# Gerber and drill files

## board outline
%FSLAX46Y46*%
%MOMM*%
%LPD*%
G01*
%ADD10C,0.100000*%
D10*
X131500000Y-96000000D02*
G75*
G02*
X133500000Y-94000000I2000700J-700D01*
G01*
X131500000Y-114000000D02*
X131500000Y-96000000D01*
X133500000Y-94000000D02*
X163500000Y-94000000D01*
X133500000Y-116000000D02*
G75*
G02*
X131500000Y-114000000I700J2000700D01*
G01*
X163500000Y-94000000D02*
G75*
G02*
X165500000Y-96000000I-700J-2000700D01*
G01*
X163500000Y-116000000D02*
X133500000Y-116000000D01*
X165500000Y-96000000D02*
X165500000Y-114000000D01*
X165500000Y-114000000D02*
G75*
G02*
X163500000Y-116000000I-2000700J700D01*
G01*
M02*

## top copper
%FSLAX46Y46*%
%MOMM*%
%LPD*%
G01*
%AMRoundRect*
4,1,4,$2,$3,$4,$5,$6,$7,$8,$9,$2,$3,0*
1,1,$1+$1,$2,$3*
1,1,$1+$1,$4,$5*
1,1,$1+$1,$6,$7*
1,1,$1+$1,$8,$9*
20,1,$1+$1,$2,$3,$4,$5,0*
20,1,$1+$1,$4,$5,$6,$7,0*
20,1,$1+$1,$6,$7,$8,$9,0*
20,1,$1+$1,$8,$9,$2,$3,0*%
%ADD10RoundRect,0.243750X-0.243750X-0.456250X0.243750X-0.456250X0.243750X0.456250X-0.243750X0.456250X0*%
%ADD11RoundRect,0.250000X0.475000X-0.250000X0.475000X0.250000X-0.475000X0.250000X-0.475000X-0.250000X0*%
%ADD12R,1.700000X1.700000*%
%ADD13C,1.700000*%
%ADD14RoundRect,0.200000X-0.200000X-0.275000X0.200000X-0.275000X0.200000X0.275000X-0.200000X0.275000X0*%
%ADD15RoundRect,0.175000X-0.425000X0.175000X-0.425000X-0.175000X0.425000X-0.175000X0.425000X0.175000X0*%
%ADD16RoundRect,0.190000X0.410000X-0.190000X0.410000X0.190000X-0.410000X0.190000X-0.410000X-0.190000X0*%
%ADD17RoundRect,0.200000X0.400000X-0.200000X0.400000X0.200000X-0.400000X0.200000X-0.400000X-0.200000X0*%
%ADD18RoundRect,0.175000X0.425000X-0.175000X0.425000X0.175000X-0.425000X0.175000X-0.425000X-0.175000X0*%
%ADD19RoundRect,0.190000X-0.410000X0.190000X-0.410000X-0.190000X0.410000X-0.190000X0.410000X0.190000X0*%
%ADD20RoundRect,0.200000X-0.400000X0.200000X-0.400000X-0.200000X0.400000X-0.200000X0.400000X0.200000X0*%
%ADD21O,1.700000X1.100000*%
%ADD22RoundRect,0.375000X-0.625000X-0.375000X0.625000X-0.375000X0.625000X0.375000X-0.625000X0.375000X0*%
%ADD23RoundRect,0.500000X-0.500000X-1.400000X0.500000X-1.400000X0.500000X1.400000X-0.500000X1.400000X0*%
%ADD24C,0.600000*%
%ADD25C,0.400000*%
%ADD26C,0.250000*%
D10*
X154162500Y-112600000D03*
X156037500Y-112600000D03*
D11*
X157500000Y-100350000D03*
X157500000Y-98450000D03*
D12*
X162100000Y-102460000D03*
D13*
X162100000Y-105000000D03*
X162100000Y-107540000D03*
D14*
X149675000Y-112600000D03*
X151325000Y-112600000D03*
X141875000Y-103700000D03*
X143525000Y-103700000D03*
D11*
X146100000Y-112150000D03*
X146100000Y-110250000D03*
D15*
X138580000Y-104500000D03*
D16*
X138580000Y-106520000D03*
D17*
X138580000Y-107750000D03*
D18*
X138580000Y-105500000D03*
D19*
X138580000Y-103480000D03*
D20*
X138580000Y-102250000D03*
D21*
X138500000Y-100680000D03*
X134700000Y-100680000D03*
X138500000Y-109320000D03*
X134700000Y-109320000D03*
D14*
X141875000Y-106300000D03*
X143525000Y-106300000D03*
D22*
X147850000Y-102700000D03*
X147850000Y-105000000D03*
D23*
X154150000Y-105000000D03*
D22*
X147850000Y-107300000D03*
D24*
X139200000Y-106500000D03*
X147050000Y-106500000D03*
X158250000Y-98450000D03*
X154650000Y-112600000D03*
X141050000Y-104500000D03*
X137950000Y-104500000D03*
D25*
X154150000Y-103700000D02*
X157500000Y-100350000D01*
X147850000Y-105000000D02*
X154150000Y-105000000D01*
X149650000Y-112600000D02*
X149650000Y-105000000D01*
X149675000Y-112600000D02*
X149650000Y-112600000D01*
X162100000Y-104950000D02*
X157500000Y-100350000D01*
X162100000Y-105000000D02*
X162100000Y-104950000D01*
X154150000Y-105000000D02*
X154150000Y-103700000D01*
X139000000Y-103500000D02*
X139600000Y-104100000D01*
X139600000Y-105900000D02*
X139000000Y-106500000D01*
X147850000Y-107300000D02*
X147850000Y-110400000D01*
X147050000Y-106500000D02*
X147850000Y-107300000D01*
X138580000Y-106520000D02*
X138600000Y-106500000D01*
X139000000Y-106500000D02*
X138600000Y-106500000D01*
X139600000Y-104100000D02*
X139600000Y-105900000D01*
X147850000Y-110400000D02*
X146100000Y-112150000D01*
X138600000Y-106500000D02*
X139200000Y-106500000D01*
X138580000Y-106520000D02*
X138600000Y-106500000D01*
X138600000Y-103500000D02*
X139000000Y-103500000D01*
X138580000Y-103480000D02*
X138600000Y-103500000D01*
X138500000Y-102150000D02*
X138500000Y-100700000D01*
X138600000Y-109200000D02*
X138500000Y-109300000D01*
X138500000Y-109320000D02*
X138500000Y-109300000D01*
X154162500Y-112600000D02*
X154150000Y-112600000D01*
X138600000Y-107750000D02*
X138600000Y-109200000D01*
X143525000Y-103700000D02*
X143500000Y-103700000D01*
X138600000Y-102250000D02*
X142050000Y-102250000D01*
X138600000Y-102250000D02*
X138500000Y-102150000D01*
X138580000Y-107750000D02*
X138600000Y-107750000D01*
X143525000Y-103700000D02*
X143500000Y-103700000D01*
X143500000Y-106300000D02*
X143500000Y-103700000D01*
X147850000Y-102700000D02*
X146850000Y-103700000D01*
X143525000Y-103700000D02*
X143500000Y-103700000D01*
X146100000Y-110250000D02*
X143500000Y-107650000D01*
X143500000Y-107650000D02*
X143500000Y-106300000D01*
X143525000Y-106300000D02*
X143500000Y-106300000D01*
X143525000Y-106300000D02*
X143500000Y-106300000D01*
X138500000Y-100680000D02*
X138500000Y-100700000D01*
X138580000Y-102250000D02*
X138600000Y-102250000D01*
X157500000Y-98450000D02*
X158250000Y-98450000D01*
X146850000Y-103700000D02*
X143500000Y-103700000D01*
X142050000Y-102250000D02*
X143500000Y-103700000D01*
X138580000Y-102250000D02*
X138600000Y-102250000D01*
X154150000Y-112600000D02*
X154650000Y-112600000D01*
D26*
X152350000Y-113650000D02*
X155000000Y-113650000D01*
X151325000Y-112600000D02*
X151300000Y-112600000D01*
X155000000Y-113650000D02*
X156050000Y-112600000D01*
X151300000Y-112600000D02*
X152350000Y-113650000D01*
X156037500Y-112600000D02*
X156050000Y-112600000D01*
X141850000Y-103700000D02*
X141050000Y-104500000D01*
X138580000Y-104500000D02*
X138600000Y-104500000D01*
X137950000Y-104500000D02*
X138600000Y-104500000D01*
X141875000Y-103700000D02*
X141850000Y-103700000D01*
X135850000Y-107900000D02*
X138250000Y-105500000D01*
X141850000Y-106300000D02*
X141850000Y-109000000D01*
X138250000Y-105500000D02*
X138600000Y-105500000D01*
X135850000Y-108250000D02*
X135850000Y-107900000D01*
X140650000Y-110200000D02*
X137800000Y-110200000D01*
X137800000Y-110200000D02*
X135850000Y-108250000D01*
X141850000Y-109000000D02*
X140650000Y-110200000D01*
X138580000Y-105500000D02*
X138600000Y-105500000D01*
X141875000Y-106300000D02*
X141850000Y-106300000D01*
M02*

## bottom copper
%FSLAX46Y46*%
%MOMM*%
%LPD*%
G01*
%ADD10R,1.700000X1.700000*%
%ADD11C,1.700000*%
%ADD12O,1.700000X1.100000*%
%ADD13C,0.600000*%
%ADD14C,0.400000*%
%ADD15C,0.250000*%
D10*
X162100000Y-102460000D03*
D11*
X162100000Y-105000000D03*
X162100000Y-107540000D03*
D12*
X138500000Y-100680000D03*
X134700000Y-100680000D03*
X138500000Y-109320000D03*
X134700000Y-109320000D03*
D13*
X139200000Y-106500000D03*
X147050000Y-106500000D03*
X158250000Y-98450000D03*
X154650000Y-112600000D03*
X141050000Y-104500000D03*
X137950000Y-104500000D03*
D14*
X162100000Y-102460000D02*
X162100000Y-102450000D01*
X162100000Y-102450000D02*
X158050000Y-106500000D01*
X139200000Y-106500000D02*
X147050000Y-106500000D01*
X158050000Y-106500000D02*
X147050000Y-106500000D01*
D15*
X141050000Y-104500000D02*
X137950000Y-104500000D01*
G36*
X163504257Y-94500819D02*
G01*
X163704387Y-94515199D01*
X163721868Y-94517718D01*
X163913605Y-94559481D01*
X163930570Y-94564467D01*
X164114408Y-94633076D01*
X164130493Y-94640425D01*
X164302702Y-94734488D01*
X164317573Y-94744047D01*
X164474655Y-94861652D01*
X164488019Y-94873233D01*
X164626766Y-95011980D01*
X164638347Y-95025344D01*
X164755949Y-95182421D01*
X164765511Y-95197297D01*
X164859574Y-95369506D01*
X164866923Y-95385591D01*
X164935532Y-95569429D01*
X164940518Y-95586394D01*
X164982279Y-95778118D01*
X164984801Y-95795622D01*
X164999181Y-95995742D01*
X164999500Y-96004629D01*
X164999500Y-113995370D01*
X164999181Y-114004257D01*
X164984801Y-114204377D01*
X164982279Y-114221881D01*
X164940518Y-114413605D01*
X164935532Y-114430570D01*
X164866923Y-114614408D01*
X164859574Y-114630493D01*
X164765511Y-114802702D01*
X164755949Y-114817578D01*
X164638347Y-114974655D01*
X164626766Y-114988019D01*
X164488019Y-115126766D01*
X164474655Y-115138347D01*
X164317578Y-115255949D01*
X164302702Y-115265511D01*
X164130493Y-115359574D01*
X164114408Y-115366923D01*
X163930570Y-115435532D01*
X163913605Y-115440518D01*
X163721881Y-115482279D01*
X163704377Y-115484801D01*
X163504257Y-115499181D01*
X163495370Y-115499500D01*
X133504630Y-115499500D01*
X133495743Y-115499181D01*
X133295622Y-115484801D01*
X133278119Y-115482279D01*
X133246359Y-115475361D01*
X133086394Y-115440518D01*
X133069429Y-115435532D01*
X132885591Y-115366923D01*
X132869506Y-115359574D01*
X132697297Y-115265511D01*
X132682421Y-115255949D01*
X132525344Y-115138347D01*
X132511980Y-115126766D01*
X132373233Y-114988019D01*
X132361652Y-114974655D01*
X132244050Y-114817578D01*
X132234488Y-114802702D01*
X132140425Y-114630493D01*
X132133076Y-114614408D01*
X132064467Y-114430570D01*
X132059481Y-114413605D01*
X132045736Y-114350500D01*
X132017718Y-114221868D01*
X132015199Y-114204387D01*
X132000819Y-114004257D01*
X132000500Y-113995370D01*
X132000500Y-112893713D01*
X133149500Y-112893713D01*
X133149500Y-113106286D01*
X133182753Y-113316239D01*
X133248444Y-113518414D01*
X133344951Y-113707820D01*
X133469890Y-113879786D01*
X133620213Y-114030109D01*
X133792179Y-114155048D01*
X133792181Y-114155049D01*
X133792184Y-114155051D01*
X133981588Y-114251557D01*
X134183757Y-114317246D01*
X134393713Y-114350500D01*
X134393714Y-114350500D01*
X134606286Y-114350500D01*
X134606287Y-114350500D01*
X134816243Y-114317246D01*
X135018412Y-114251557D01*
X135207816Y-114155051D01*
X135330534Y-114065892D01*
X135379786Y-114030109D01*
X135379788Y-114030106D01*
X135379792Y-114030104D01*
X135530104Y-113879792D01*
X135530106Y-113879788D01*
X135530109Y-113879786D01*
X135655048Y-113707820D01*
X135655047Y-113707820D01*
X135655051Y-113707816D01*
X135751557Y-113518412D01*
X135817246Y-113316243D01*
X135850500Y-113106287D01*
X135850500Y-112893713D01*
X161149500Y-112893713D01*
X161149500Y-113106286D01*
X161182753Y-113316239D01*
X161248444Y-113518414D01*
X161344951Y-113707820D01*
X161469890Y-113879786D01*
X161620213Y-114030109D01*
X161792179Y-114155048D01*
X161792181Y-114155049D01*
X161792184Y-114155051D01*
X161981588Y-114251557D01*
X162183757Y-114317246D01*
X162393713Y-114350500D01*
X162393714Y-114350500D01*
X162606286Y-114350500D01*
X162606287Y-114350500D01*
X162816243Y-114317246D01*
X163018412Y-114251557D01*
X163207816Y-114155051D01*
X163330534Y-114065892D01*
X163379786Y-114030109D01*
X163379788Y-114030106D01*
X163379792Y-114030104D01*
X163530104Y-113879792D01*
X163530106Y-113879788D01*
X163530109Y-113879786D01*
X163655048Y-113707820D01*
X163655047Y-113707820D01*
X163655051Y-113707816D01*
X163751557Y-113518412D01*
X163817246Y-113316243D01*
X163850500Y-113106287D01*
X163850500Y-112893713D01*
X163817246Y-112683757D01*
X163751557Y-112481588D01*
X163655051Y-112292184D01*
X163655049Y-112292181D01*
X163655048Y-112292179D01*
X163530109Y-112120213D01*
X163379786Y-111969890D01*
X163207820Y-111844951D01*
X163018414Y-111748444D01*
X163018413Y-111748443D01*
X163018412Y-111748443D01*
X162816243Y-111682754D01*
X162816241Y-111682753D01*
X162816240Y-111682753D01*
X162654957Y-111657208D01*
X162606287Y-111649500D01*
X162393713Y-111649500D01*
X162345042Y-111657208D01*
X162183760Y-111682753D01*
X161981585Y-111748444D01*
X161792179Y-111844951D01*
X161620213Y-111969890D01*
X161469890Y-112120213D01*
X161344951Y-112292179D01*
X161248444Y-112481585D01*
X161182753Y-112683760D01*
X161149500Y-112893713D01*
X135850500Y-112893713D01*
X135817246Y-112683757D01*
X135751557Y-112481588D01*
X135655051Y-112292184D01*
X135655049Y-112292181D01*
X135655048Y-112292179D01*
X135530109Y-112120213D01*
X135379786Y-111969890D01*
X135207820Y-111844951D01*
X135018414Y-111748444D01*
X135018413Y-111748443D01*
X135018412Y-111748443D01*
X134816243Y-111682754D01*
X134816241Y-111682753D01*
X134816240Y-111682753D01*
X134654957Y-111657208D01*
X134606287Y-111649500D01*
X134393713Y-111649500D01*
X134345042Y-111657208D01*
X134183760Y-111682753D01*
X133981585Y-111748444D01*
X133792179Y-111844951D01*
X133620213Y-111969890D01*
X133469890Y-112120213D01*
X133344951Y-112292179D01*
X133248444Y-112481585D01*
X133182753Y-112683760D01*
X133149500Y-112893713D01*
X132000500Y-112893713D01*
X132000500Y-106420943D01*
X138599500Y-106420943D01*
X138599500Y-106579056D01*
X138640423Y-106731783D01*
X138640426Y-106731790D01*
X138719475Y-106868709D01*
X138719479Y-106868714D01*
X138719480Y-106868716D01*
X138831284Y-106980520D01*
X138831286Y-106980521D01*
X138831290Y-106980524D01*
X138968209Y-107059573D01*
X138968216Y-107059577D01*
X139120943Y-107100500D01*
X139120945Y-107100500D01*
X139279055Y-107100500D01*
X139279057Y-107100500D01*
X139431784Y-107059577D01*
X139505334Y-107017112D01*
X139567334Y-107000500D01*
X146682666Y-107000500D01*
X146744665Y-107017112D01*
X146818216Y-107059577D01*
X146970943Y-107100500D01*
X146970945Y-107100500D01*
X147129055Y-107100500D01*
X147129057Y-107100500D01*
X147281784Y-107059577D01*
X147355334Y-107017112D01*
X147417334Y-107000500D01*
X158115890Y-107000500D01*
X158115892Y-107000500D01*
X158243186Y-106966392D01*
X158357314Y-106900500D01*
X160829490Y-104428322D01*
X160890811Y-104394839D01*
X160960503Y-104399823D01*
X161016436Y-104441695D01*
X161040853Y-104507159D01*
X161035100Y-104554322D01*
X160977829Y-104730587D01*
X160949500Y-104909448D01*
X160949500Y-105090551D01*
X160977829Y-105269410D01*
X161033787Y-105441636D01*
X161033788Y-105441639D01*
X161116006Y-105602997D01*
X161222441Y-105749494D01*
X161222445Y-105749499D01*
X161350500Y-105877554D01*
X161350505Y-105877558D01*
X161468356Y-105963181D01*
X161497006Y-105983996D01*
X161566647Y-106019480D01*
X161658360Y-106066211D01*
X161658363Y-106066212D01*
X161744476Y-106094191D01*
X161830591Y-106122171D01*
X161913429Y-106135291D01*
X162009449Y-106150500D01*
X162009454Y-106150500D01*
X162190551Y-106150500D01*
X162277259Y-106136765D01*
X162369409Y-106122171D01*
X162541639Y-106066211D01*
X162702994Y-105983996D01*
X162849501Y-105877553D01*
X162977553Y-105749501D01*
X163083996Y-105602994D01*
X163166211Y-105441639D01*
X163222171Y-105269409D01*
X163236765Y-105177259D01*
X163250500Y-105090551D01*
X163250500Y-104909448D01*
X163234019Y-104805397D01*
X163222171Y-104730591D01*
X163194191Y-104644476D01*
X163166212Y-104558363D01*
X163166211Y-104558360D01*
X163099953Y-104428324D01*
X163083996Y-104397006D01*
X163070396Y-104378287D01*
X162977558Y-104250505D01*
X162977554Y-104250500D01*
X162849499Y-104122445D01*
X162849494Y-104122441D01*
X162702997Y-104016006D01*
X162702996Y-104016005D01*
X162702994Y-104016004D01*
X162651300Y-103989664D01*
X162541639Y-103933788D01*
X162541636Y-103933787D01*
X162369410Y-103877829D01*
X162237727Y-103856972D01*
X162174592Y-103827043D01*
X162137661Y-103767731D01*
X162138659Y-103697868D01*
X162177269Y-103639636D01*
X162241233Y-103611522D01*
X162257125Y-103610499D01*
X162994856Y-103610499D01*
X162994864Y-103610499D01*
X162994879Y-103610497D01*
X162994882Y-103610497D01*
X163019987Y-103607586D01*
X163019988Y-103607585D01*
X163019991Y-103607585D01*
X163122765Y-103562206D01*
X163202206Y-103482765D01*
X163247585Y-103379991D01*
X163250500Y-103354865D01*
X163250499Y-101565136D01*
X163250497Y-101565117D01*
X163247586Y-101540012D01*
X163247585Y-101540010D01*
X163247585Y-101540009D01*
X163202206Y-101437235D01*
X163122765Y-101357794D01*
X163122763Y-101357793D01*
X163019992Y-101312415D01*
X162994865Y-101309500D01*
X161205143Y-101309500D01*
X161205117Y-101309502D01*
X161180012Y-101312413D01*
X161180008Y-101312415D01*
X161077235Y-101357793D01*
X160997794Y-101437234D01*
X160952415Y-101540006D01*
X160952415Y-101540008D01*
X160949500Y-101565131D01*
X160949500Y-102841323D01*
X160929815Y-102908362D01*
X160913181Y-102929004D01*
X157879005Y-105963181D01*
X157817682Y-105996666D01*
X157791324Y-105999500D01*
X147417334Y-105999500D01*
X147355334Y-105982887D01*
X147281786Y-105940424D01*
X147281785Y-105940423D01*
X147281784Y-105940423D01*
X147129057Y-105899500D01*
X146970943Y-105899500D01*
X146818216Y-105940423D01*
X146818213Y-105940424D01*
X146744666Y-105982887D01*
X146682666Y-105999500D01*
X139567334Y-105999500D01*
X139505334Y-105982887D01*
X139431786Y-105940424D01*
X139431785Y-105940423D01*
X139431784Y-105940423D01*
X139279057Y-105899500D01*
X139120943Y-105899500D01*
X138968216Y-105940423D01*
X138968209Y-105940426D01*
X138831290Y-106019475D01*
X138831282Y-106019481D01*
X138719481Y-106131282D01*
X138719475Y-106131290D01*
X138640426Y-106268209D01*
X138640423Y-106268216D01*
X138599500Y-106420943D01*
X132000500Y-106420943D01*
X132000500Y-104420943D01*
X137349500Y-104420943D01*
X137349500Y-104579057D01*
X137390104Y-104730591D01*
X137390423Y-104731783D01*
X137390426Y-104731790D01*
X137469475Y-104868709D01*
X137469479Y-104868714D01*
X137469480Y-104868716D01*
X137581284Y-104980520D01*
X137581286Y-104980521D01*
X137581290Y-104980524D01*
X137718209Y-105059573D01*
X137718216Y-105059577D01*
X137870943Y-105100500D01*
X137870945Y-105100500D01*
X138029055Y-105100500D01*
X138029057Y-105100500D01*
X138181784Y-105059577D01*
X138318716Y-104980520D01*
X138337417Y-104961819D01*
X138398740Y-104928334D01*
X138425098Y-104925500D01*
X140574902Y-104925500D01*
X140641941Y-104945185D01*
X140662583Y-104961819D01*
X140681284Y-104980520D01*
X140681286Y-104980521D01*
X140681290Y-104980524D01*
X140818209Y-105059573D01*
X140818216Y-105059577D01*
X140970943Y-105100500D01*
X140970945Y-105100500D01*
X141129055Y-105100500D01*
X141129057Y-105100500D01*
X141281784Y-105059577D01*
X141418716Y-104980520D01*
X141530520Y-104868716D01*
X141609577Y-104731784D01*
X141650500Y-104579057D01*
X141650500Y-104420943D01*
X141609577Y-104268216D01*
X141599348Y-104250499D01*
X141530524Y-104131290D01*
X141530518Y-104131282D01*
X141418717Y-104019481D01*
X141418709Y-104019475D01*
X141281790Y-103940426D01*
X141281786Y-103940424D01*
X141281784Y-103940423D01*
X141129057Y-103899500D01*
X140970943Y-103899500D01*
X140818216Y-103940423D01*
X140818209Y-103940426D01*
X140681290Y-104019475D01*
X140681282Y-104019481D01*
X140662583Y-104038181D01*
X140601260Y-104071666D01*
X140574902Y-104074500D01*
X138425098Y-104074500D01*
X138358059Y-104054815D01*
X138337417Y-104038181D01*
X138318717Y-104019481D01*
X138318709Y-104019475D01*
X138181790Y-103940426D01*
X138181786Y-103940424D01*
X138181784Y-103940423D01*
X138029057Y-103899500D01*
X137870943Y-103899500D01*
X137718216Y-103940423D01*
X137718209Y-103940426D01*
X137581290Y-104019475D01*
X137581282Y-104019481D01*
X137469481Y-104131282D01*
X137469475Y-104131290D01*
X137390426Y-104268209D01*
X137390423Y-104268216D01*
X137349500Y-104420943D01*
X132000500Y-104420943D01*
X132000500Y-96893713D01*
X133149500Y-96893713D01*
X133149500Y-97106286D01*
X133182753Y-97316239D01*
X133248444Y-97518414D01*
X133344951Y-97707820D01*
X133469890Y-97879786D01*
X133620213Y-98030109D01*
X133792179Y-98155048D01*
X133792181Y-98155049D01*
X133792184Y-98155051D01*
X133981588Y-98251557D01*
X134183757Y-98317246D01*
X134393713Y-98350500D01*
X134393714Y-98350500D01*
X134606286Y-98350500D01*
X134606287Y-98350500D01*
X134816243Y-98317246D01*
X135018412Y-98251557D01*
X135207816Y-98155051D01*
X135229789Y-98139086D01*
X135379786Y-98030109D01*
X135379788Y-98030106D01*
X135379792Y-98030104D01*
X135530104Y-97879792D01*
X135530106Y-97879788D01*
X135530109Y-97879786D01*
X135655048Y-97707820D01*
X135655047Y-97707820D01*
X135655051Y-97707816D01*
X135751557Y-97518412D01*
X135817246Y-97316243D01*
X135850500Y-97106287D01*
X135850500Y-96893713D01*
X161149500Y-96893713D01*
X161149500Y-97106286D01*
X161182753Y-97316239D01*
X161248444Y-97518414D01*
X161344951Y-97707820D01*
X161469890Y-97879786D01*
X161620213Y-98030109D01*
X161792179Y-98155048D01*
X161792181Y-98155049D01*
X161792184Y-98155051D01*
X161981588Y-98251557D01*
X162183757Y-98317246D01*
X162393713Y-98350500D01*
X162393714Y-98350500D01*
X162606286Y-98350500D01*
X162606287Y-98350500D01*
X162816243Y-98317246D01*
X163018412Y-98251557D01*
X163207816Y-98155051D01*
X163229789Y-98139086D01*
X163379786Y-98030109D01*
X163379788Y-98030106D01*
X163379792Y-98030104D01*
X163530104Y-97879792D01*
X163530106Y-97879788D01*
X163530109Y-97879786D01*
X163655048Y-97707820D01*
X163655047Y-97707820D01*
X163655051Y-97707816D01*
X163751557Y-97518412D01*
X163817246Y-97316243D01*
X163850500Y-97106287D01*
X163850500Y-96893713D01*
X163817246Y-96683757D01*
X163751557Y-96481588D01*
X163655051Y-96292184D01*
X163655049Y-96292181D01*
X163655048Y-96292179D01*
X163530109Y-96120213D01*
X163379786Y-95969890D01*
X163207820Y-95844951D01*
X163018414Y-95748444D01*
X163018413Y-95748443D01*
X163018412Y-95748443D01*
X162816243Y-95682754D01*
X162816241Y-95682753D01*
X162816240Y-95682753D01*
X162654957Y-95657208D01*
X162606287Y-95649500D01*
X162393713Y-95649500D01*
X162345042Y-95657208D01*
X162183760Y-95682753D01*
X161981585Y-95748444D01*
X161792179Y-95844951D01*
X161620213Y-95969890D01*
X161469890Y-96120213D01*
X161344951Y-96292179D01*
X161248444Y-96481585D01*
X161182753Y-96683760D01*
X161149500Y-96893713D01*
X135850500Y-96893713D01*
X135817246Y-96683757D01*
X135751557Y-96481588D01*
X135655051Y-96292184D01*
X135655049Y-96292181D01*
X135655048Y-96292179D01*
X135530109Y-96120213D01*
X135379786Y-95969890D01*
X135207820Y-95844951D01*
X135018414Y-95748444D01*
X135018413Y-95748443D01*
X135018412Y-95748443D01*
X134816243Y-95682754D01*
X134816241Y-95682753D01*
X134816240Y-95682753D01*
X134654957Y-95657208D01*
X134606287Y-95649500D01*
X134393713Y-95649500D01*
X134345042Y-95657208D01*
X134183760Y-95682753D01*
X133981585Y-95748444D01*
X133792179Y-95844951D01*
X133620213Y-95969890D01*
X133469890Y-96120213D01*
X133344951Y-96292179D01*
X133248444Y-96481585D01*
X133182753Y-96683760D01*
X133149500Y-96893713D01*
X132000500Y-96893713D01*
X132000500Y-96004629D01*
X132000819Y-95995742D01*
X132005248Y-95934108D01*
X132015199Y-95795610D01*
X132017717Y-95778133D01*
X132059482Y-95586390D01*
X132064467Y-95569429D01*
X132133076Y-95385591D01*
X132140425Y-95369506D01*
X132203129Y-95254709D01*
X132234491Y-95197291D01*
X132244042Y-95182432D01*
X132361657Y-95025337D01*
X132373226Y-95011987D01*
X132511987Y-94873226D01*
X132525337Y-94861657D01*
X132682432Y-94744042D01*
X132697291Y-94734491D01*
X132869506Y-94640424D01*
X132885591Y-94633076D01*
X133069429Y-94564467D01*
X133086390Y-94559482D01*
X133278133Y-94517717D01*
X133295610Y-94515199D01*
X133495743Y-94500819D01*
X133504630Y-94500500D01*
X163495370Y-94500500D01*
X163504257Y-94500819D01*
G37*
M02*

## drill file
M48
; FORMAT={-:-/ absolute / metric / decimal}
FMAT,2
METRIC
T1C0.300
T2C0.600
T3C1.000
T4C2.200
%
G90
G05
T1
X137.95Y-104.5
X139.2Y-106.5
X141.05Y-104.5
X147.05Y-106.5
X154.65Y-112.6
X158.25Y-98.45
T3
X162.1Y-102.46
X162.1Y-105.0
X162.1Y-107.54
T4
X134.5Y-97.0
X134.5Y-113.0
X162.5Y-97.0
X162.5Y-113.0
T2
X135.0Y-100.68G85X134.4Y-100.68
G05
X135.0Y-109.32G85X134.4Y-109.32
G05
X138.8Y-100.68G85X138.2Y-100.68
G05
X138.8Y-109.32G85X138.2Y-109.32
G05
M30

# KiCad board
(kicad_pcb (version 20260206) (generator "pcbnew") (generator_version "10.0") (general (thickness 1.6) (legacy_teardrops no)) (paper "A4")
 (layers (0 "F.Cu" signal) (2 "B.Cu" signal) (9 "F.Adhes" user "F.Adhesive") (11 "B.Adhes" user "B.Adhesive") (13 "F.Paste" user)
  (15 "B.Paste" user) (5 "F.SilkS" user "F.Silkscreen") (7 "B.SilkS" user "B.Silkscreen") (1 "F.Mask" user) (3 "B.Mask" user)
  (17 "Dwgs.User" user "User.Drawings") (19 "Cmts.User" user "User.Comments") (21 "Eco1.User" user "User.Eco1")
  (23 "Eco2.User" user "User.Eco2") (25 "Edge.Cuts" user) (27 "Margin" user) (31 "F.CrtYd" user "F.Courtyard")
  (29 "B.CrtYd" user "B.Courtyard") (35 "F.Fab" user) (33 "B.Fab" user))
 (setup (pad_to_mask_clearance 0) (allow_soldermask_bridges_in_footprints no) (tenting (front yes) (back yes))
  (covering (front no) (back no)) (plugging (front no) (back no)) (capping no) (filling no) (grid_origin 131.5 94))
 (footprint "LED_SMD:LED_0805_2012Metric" (layer "F.Cu") (at 155.1 112.6)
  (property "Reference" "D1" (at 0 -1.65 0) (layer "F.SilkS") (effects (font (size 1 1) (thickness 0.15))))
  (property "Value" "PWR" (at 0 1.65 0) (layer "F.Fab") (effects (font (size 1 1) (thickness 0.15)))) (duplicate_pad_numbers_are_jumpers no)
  (pad "1" smd roundrect (at -0.9375 0) (size 0.975 1.4) (layers "F.Cu" "F.Mask" "F.Paste") (roundrect_rratio 0.25) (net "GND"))
  (pad "2" smd roundrect (at 0.9375 0) (size 0.975 1.4) (layers "F.Cu" "F.Mask" "F.Paste") (roundrect_rratio 0.25) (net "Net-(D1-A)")))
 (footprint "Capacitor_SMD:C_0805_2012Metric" (layer "F.Cu") (at 157.5 99.4 90)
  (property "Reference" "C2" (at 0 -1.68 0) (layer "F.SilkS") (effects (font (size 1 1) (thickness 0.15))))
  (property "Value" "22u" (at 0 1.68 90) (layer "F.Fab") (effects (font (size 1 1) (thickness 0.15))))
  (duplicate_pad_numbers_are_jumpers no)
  (pad "1" smd roundrect (at -0.95 0 90) (size 1 1.45) (layers "F.Cu" "F.Mask" "F.Paste") (roundrect_rratio 0.25) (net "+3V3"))
  (pad "2" smd roundrect (at 0.95 0 90) (size 1 1.45) (layers "F.Cu" "F.Mask" "F.Paste") (roundrect_rratio 0.25) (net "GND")))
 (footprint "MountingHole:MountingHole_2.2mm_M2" (layer "F.Cu") (at 162.5 97)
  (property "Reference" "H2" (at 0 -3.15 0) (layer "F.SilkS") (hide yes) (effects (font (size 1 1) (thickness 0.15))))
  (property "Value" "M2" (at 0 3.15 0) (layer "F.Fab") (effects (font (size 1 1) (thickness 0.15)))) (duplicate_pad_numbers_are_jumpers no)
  (pad "" np_thru_hole circle (at 0 0) (size 2.2 2.2) (drill 2.2) (layers "*.Cu" "*.Mask")))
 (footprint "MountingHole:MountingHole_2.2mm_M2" (layer "F.Cu") (at 134.5 97)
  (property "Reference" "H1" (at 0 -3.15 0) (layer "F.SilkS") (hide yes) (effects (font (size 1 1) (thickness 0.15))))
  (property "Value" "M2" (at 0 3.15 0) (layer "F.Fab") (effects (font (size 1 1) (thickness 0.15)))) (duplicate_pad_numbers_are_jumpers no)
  (pad "" np_thru_hole circle (at 0 0) (size 2.2 2.2) (drill 2.2) (layers "*.Cu" "*.Mask")))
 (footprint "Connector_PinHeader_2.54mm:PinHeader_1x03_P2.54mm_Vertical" (layer "F.Cu") (at 162.1 102.46)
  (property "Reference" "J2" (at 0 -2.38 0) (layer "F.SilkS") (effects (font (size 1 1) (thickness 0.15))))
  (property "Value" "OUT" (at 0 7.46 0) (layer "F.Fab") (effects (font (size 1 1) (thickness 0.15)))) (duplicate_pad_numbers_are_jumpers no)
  (pad "1" thru_hole rect (at 0 0) (size 1.7 1.7) (drill 1) (layers "*.Cu" "*.Mask") (remove_unused_layers no) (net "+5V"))
  (pad "2" thru_hole circle (at 0 2.54) (size 1.7 1.7) (drill 1) (layers "*.Cu" "*.Mask") (remove_unused_layers no) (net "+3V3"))
  (pad "3" thru_hole circle (at 0 5.08) (size 1.7 1.7) (drill 1) (layers "*.Cu" "*.Mask") (remove_unused_layers no) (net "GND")))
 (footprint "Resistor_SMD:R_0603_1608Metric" (layer "F.Cu") (at 150.5 112.6)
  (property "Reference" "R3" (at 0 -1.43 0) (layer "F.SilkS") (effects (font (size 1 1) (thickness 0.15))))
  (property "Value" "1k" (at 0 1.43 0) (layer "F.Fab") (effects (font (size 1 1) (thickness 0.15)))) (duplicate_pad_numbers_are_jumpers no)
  (pad "1" smd roundrect (at -0.825 0) (size 0.8 0.95) (layers "F.Cu" "F.Mask" "F.Paste") (roundrect_rratio 0.25) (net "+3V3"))
  (pad "2" smd roundrect (at 0.825 0) (size 0.8 0.95) (layers "F.Cu" "F.Mask" "F.Paste") (roundrect_rratio 0.25) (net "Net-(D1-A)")))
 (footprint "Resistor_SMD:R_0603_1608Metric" (layer "F.Cu") (at 142.7 103.7)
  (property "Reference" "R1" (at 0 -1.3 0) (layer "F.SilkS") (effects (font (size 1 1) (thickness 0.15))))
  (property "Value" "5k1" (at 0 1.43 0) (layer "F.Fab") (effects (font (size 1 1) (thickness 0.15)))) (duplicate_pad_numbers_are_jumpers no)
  (pad "1" smd roundrect (at -0.825 0) (size 0.8 0.95) (layers "F.Cu" "F.Mask" "F.Paste") (roundrect_rratio 0.25) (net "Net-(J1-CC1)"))
  (pad "2" smd roundrect (at 0.825 0) (size 0.8 0.95) (layers "F.Cu" "F.Mask" "F.Paste") (roundrect_rratio 0.25) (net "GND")))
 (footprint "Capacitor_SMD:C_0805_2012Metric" (layer "F.Cu") (at 146.1 111.2 90)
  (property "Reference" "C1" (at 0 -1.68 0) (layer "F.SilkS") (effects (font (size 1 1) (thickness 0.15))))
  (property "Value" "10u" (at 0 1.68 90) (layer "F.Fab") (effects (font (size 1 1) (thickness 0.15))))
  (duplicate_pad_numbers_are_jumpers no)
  (pad "1" smd roundrect (at -0.95 0 90) (size 1 1.45) (layers "F.Cu" "F.Mask" "F.Paste") (roundrect_rratio 0.25) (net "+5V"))
  (pad "2" smd roundrect (at 0.95 0 90) (size 1 1.45) (layers "F.Cu" "F.Mask" "F.Paste") (roundrect_rratio 0.25) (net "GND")))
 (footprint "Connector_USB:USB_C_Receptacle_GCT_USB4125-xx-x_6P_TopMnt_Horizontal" (layer "F.Cu") (at 135.5 105 -90)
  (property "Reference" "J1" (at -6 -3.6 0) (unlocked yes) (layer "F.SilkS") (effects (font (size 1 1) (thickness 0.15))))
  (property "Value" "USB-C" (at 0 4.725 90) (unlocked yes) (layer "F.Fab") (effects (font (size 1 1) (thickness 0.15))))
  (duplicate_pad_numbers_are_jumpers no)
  (pad "A5" smd roundrect (at -0.5 -3.08 270) (size 0.7 1.2) (layers "F.Cu" "F.Mask" "F.Paste") (roundrect_rratio 0.25) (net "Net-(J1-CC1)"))
  (pad "A9" smd roundrect (at 1.52 -3.08 90) (size 0.76 1.2) (layers "F.Cu" "F.Mask" "F.Paste") (roundrect_rratio 0.25) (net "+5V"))
  (pad "A12" smd roundrect (at 2.75 -3.08 90) (size 0.8 1.2) (layers "F.Cu" "F.Mask" "F.Paste") (roundrect_rratio 0.25) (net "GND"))
  (pad "B5" smd roundrect (at 0.5 -3.08 90) (size 0.7 1.2) (layers "F.Cu" "F.Mask" "F.Paste") (roundrect_rratio 0.25) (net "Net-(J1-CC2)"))
  (pad "B9" smd roundrect (at -1.52 -3.08 270) (size 0.76 1.2) (layers "F.Cu" "F.Mask" "F.Paste") (roundrect_rratio 0.25) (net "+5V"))
  (pad "B12" smd roundrect (at -2.75 -3.08 270) (size 0.8 1.2) (layers "F.Cu" "F.Mask" "F.Paste") (roundrect_rratio 0.25) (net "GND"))
  (pad "SH" thru_hole oval (at -4.32 -3 270) (size 1.1 1.7) (drill oval 0.6 1.2) (layers "*.Cu" "*.Mask" "F.Paste")
   (remove_unused_layers no) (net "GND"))
  (pad "SH" thru_hole oval (at -4.32 0.8 270) (size 1.1 1.7) (drill oval 0.6 1.2) (layers "*.Cu" "*.Mask" "F.Paste")
   (remove_unused_layers no) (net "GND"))
  (pad "SH" thru_hole oval (at 4.32 -3 270) (size 1.1 1.7) (drill oval 0.6 1.2) (layers "*.Cu" "*.Mask" "F.Paste") (remove_unused_layers no)
   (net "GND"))
  (pad "SH" thru_hole oval (at 4.32 0.8 270) (size 1.1 1.7) (drill oval 0.6 1.2) (layers "*.Cu" "*.Mask" "F.Paste")
   (remove_unused_layers no) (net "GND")))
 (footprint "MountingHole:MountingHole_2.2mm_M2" (layer "F.Cu") (at 134.5 113)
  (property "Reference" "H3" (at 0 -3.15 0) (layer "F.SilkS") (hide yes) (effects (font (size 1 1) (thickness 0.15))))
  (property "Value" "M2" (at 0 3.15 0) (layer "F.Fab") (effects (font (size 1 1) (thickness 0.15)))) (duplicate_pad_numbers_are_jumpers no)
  (pad "" np_thru_hole circle (at 0 0) (size 2.2 2.2) (drill 2.2) (layers "*.Cu" "*.Mask")))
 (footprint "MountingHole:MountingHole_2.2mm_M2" (layer "F.Cu") (at 162.5 113)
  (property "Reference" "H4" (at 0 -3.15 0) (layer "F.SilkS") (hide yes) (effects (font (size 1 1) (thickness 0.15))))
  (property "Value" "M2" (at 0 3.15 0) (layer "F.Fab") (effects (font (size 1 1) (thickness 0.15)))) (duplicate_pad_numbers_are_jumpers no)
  (pad "" np_thru_hole circle (at 0 0) (size 2.2 2.2) (drill 2.2) (layers "*.Cu" "*.Mask")))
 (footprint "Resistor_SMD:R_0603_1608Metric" (layer "F.Cu") (at 142.7 106.3)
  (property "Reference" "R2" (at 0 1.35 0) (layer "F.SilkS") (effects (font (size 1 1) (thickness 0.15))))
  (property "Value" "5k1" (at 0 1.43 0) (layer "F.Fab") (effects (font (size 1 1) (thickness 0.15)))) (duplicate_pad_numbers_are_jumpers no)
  (pad "1" smd roundrect (at -0.825 0) (size 0.8 0.95) (layers "F.Cu" "F.Mask" "F.Paste") (roundrect_rratio 0.25) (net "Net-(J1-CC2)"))
  (pad "2" smd roundrect (at 0.825 0) (size 0.8 0.95) (layers "F.Cu" "F.Mask" "F.Paste") (roundrect_rratio 0.25) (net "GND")))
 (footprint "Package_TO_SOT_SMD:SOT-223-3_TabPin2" (layer "F.Cu") (at 151 105)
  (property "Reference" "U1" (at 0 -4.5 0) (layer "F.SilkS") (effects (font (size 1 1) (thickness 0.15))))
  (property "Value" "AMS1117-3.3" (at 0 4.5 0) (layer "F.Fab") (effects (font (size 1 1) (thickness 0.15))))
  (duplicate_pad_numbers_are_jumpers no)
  (pad "1" smd roundrect (at -3.15 -2.3) (size 2 1.5) (layers "F.Cu" "F.Mask" "F.Paste") (roundrect_rratio 0.25) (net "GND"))
  (pad "2" smd roundrect (at -3.15 0) (size 2 1.5) (layers "F.Cu" "F.Mask" "F.Paste") (roundrect_rratio 0.25) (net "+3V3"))
  (pad "2" smd roundrect (at 3.15 0) (size 2 3.8) (layers "F.Cu" "F.Mask" "F.Paste") (roundrect_rratio 0.25) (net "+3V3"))
  (pad "3" smd roundrect (at -3.15 2.3) (size 2 1.5) (layers "F.Cu" "F.Mask" "F.Paste") (roundrect_rratio 0.25) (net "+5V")))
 (gr_arc (start 131.5 96) (mid 132.086 94.586) (end 133.5 94) (stroke (width 0.1) (type default)) (layer "Edge.Cuts"))
 (gr_line (start 131.5 114) (end 131.5 96) (stroke (width 0.1) (type default)) (layer "Edge.Cuts"))
 (gr_line (start 133.5 94) (end 163.5 94) (stroke (width 0.1) (type default)) (layer "Edge.Cuts"))
 (gr_arc (start 133.5 116) (mid 132.086 115.414) (end 131.5 114) (stroke (width 0.1) (type default)) (layer "Edge.Cuts"))
 (gr_arc (start 163.5 94) (mid 164.914 94.586) (end 165.5 96) (stroke (width 0.1) (type default)) (layer "Edge.Cuts"))
 (gr_line (start 163.5 116) (end 133.5 116) (stroke (width 0.1) (type default)) (layer "Edge.Cuts"))
 (gr_line (start 165.5 96) (end 165.5 114) (stroke (width 0.1) (type default)) (layer "Edge.Cuts"))
 (gr_arc (start 165.5 114) (mid 164.914 115.414) (end 163.5 116) (stroke (width 0.1) (type default)) (layer "Edge.Cuts"))
 (segment (start 154.15 103.7) (end 157.5 100.35) (width 0.4) (layer "F.Cu") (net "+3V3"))
 (segment (start 147.85 105) (end 154.15 105) (width 0.4) (layer "F.Cu") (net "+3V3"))
 (segment (start 149.65 112.6) (end 149.65 105) (width 0.4) (layer "F.Cu") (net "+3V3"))
 (segment (start 149.675 112.6) (end 149.65 112.6) (width 0.4) (layer "F.Cu") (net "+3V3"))
 (segment (start 162.1 104.95) (end 157.5 100.35) (width 0.4) (layer "F.Cu") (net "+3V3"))
 (segment (start 162.1 105) (end 162.1 104.95) (width 0.4) (layer "F.Cu") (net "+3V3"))
 (segment (start 154.15 105) (end 154.15 103.7) (width 0.4) (layer "F.Cu") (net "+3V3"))
 (segment (start 139 103.5) (end 139.6 104.1) (width 0.4) (layer "F.Cu") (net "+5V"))
 (segment (start 139.6 105.9) (end 139 106.5) (width 0.4) (layer "F.Cu") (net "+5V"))
 (segment (start 147.85 107.3) (end 147.85 110.4) (width 0.4) (layer "F.Cu") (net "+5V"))
 (segment (start 147.05 106.5) (end 147.85 107.3) (width 0.4) (layer "F.Cu") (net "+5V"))
 (segment (start 138.58 106.52) (end 138.6 106.5) (width 0.4) (layer "F.Cu") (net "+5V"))
 (segment (start 139 106.5) (end 138.6 106.5) (width 0.4) (layer "F.Cu") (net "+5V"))
 (segment (start 139.6 104.1) (end 139.6 105.9) (width 0.4) (layer "F.Cu") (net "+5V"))
 (segment (start 147.85 110.4) (end 146.1 112.15) (width 0.4) (layer "F.Cu") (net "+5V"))
 (segment (start 138.6 106.5) (end 139.2 106.5) (width 0.4) (layer "F.Cu") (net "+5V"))
 (segment (start 138.58 106.52) (end 138.6 106.5) (width 0.4) (layer "F.Cu") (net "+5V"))
 (segment (start 138.6 103.5) (end 139 103.5) (width 0.4) (layer "F.Cu") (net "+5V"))
 (segment (start 138.58 103.48) (end 138.6 103.5) (width 0.4) (layer "F.Cu") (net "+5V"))
 (via (at 139.2 106.5) (size 0.6) (drill 0.3) (layers "F.Cu" "B.Cu") (capping no) (covering (front no) (back no))
  (plugging (front no) (back no)) (filling no) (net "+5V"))
 (via (at 147.05 106.5) (size 0.6) (drill 0.3) (layers "F.Cu" "B.Cu") (capping no) (covering (front no) (back no))
  (plugging (front no) (back no)) (filling no) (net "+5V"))
 (segment (start 162.1 102.46) (end 162.1 102.45) (width 0.4) (layer "B.Cu") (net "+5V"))
 (segment (start 162.1 102.45) (end 158.05 106.5) (width 0.4) (layer "B.Cu") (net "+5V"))
 (segment (start 139.2 106.5) (end 147.05 106.5) (width 0.4) (layer "B.Cu") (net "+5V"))
 (segment (start 158.05 106.5) (end 147.05 106.5) (width 0.4) (layer "B.Cu") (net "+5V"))
 (segment (start 138.5 102.15) (end 138.5 100.7) (width 0.4) (layer "F.Cu") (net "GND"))
 (segment (start 138.6 109.2) (end 138.5 109.3) (width 0.4) (layer "F.Cu") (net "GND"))
 (segment (start 138.5 109.32) (end 138.5 109.3) (width 0.4) (layer "F.Cu") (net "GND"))
 (segment (start 154.1625 112.6) (end 154.15 112.6) (width 0.4) (layer "F.Cu") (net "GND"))
 (segment (start 138.6 107.75) (end 138.6 109.2) (width 0.4) (layer "F.Cu") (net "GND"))
 (segment (start 143.525 103.7) (end 143.5 103.7) (width 0.4) (layer "F.Cu") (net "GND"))
 (segment (start 138.6 102.25) (end 142.05 102.25) (width 0.4) (layer "F.Cu") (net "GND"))
 (segment (start 138.6 102.25) (end 138.5 102.15) (width 0.4) (layer "F.Cu") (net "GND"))
 (segment (start 138.58 107.75) (end 138.6 107.75) (width 0.4) (layer "F.Cu") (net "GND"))
 (segment (start 143.525 103.7) (end 143.5 103.7) (width 0.4) (layer "F.Cu") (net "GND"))
 (segment (start 143.5 106.3) (end 143.5 103.7) (width 0.4) (layer "F.Cu") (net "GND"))
 (segment (start 147.85 102.7) (end 146.85 103.7) (width 0.4) (layer "F.Cu") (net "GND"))
 (segment (start 143.525 103.7) (end 143.5 103.7) (width 0.4) (layer "F.Cu") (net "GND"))
 (segment (start 146.1 110.25) (end 143.5 107.65) (width 0.4) (layer "F.Cu") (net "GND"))
 (segment (start 143.5 107.65) (end 143.5 106.3) (width 0.4) (layer "F.Cu") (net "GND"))
 (segment (start 143.525 106.3) (end 143.5 106.3) (width 0.4) (layer "F.Cu") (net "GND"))
 (segment (start 143.525 106.3) (end 143.5 106.3) (width 0.4) (layer "F.Cu") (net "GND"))
 (segment (start 138.5 100.68) (end 138.5 100.7) (width 0.4) (layer "F.Cu") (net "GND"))
 (segment (start 138.58 102.25) (end 138.6 102.25) (width 0.4) (layer "F.Cu") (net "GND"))
 (segment (start 157.5 98.45) (end 158.25 98.45) (width 0.4) (layer "F.Cu") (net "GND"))
 (segment (start 146.85 103.7) (end 143.5 103.7) (width 0.4) (layer "F.Cu") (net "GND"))
 (segment (start 142.05 102.25) (end 143.5 103.7) (width 0.4) (layer "F.Cu") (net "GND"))
 (segment (start 138.58 102.25) (end 138.6 102.25) (width 0.4) (layer "F.Cu") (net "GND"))
 (segment (start 154.15 112.6) (end 154.65 112.6) (width 0.4) (layer "F.Cu") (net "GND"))
 (via (at 158.25 98.45) (size 0.6) (drill 0.3) (layers "F.Cu" "B.Cu") (capping no) (covering (front no) (back no))
  (plugging (front no) (back no)) (filling no) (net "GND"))
 (via (at 154.65 112.6) (size 0.6) (drill 0.3) (layers "F.Cu" "B.Cu") (capping no) (covering (front no) (back no))
  (plugging (front no) (back no)) (filling no) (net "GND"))
 (segment (start 152.35 113.65) (end 155 113.65) (width 0.25) (layer "F.Cu") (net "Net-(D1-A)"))
 (segment (start 151.325 112.6) (end 151.3 112.6) (width 0.25) (layer "F.Cu") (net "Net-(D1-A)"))
 (segment (start 155 113.65) (end 156.05 112.6) (width 0.25) (layer "F.Cu") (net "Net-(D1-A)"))
 (segment (start 151.3 112.6) (end 152.35 113.65) (width 0.25) (layer "F.Cu") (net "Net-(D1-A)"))
 (segment (start 156.0375 112.6) (end 156.05 112.6) (width 0.25) (layer "F.Cu") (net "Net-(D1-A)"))
 (segment (start 141.85 103.7) (end 141.05 104.5) (width 0.25) (layer "F.Cu") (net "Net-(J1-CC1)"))
 (segment (start 138.58 104.5) (end 138.6 104.5) (width 0.25) (layer "F.Cu") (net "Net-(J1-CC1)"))
 (segment (start 137.95 104.5) (end 138.6 104.5) (width 0.25) (layer "F.Cu") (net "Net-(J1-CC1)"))
 (segment (start 141.875 103.7) (end 141.85 103.7) (width 0.25) (layer "F.Cu") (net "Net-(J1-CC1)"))
 (via (at 141.05 104.5) (size 0.6) (drill 0.3) (layers "F.Cu" "B.Cu") (capping no) (covering (front no) (back no))
  (plugging (front no) (back no)) (filling no) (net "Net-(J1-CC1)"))
 (via (at 137.95 104.5) (size 0.6) (drill 0.3) (layers "F.Cu" "B.Cu") (capping no) (covering (front no) (back no))
  (plugging (front no) (back no)) (filling no) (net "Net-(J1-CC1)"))
 (segment (start 141.05 104.5) (end 137.95 104.5) (width 0.25) (layer "B.Cu") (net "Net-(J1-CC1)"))
 (segment (start 135.85 107.9) (end 138.25 105.5) (width 0.25) (layer "F.Cu") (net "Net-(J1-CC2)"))
 (segment (start 141.85 106.3) (end 141.85 109) (width 0.25) (layer "F.Cu") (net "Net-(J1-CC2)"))
 (segment (start 138.25 105.5) (end 138.6 105.5) (width 0.25) (layer "F.Cu") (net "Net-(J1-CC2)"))
 (segment (start 135.85 108.25) (end 135.85 107.9) (width 0.25) (layer "F.Cu") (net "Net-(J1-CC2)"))
 (segment (start 140.65 110.2) (end 137.8 110.2) (width 0.25) (layer "F.Cu") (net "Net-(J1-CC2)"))
 (segment (start 137.8 110.2) (end 135.85 108.25) (width 0.25) (layer "F.Cu") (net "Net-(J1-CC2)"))
 (segment (start 141.85 109) (end 140.65 110.2) (width 0.25) (layer "F.Cu") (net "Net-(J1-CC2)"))
 (segment (start 138.58 105.5) (end 138.6 105.5) (width 0.25) (layer "F.Cu") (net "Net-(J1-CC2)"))
 (segment (start 141.875 106.3) (end 141.85 106.3) (width 0.25) (layer "F.Cu") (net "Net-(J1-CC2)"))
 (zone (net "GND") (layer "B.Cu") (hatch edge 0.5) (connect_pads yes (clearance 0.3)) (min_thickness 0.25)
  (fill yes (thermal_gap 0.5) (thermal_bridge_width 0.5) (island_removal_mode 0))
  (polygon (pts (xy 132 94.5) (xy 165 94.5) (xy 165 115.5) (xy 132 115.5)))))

